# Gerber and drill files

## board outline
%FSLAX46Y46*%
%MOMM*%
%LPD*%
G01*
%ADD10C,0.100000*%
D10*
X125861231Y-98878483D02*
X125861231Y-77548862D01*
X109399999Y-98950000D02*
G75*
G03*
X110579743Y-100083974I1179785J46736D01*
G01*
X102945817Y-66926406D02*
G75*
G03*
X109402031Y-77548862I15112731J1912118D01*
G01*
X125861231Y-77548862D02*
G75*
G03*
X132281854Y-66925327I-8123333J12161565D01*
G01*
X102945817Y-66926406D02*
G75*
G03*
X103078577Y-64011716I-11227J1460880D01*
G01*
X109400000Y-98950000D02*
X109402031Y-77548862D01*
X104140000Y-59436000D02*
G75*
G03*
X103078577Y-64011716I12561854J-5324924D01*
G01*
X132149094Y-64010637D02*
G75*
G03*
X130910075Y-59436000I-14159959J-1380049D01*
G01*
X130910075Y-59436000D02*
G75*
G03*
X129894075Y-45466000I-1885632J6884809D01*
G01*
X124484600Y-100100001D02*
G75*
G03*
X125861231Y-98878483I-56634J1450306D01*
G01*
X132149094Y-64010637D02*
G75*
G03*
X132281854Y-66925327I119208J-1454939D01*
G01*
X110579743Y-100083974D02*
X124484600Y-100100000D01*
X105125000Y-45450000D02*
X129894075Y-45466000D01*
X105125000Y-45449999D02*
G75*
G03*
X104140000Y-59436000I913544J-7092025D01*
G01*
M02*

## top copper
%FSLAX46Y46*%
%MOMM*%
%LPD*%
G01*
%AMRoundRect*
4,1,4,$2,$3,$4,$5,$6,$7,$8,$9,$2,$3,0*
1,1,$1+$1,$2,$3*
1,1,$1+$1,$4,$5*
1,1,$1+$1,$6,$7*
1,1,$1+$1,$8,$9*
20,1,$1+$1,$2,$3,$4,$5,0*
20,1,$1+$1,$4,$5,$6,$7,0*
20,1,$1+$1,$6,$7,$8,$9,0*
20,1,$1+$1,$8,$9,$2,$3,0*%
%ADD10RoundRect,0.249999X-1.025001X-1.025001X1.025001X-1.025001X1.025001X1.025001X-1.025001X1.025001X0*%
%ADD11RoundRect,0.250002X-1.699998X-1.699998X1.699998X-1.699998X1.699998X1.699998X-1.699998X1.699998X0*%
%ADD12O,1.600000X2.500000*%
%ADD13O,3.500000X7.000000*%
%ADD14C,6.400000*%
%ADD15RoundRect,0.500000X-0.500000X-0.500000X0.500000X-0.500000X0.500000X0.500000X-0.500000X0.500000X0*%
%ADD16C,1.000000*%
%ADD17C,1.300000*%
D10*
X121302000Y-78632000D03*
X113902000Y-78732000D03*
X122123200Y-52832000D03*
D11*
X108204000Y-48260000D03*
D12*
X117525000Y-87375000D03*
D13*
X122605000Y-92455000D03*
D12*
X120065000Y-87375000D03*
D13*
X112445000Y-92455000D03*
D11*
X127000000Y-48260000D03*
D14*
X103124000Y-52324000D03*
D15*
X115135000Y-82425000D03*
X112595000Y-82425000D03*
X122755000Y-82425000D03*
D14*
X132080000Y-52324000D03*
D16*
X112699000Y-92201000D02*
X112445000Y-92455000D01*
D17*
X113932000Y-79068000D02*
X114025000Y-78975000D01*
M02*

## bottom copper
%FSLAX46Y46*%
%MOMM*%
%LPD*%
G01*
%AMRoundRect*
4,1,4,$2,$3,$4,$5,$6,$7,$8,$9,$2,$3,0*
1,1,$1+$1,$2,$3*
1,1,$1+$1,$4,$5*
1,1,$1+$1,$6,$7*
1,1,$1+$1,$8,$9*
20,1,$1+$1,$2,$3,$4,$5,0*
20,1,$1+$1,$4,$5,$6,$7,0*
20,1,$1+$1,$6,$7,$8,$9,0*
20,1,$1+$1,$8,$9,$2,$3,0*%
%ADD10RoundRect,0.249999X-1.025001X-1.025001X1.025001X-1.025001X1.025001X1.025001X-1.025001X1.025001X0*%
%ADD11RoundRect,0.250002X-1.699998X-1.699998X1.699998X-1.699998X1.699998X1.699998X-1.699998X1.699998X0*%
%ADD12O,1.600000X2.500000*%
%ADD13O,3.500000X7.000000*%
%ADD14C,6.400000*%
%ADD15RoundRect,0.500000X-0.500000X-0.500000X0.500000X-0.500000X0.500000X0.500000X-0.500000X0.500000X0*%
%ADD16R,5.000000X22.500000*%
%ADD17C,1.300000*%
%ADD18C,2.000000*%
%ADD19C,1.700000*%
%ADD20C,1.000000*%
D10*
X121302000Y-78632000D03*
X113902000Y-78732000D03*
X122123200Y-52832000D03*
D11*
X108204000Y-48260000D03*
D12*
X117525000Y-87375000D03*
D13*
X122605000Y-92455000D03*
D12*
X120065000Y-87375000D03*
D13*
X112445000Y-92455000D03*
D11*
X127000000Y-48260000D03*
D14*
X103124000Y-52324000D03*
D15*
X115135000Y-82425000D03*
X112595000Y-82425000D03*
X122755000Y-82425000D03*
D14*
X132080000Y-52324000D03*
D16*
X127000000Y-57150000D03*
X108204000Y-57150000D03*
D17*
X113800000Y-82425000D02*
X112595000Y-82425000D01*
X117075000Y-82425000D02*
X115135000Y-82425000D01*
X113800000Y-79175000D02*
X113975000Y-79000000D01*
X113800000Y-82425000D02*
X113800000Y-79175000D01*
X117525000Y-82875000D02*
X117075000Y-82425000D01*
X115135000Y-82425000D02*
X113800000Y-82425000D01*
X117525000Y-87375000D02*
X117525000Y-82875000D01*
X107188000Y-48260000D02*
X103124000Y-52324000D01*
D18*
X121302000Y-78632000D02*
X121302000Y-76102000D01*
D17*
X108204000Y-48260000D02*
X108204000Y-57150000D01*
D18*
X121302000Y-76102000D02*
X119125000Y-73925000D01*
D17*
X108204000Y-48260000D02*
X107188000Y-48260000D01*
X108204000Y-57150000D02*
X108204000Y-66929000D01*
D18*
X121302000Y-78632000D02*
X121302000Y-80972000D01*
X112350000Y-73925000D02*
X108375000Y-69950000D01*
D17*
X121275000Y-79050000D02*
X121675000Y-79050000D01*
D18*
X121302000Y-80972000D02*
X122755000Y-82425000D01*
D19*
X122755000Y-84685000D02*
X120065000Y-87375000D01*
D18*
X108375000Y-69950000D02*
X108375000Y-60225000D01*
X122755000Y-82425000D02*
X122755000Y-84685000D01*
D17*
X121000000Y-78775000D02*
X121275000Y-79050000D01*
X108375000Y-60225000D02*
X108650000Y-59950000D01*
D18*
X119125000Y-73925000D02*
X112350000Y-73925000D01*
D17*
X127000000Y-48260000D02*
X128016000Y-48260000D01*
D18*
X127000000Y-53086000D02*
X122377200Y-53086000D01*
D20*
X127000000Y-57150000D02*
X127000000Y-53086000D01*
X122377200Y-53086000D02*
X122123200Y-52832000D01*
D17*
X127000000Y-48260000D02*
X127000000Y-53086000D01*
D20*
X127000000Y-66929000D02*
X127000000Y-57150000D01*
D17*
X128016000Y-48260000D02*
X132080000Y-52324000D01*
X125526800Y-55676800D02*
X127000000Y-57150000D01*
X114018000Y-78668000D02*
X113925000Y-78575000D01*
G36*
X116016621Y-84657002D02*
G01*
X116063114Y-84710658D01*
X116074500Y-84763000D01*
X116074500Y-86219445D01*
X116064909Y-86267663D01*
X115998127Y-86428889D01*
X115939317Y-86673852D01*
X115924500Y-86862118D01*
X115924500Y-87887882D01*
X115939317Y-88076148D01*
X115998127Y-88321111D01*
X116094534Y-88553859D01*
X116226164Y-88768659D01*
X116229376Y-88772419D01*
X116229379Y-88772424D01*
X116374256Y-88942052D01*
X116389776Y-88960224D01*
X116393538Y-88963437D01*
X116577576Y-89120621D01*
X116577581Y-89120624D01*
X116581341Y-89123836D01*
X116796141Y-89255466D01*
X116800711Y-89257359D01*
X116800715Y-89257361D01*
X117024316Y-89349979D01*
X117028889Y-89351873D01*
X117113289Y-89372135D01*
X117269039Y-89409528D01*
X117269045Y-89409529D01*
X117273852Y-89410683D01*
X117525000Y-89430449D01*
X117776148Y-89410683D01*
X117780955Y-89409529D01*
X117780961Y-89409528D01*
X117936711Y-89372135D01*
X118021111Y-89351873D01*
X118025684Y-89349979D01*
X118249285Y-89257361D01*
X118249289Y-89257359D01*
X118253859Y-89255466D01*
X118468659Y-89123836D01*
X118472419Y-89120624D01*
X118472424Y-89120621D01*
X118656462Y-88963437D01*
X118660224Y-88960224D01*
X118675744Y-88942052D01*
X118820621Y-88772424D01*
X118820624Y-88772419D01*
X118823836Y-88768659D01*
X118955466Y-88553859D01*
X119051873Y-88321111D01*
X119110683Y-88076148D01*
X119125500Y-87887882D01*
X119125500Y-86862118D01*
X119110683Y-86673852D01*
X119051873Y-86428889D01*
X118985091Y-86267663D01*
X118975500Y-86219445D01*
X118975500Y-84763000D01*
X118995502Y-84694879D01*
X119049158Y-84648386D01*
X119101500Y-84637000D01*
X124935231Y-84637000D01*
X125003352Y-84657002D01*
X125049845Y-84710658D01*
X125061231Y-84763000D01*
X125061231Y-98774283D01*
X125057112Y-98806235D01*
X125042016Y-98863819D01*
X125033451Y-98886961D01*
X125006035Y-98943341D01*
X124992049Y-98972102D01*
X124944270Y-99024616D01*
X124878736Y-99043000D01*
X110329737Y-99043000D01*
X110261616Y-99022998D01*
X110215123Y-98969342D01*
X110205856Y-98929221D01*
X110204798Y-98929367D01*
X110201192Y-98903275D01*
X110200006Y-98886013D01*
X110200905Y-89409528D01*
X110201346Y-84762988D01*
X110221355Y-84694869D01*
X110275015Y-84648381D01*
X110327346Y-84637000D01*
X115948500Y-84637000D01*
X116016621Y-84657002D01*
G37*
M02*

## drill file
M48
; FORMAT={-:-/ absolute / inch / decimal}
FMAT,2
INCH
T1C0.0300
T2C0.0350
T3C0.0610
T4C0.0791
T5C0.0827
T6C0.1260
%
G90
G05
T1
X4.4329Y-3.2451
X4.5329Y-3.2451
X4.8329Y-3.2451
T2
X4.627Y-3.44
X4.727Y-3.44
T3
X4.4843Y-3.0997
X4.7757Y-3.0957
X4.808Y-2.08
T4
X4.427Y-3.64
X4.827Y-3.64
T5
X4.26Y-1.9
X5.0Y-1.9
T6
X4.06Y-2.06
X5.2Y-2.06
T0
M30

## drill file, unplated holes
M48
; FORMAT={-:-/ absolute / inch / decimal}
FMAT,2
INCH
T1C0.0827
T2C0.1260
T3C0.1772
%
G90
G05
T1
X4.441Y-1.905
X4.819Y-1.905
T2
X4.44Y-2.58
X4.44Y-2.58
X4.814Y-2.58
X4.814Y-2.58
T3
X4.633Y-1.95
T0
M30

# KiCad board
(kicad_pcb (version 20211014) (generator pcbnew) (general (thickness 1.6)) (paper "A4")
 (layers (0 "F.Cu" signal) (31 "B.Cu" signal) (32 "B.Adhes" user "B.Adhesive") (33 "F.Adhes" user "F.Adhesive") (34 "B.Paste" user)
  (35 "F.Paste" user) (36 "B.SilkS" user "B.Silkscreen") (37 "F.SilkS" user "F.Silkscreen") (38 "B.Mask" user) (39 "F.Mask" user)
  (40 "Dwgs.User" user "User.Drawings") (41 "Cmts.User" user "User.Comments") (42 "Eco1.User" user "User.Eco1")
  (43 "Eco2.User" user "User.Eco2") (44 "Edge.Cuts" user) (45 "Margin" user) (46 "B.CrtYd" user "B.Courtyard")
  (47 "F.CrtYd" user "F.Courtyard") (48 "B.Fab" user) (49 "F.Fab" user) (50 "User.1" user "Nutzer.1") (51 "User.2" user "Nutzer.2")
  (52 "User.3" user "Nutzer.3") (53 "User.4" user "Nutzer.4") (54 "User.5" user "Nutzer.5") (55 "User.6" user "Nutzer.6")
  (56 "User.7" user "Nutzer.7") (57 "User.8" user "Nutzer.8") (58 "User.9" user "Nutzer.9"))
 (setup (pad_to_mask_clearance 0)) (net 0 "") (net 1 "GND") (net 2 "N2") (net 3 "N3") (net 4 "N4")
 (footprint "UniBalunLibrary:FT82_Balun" (layer "F.Cu") (at 117.602 65.532)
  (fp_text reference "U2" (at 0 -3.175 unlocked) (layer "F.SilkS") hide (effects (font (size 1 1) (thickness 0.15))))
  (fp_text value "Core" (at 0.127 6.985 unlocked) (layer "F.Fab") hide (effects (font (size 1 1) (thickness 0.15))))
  (pad "" np_thru_hole circle (at 4.6736 0) (size 3.2 3.2) (drill 3.2) (layers *.Cu *.Mask))
  (pad "" np_thru_hole circle (at -4.826 0) (size 3.2 3.2) (drill 3.2) (layers *.Cu *.Mask))
  (pad "" np_thru_hole circle (at -4.826 0) (size 3.2 3.2) (drill 3.2) (layers *.Cu *.Mask))
  (pad "" np_thru_hole circle (at 4.6736 0) (size 3.2 3.2) (drill 3.2) (layers *.Cu *.Mask))
  (pad "1" thru_hole roundrect (at 3.7 13.1) (size 2.55 2.55) (drill 1.55) (layers *.Cu *.Mask) (roundrect_rratio 0.09803882353)
   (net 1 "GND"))
  (pad "4" thru_hole roundrect (at -3.7 13.2) (size 2.55 2.55) (drill 1.55) (layers *.Cu *.Mask) (roundrect_rratio 0.09803882353)
   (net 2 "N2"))
  (pad "5" thru_hole roundrect (at 4.5212 -12.7) (size 2.55 2.55) (drill 1.55) (layers *.Cu *.Mask) (roundrect_rratio 0.09803882353)
   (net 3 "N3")))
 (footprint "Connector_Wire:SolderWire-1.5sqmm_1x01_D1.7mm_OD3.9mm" (layer "F.Cu") (at 108.204 48.26)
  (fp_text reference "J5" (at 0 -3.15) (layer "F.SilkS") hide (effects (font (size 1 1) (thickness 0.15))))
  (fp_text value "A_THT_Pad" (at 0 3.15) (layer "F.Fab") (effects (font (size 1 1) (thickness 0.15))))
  (pad "1" thru_hole roundrect (at 0 0) (size 3.9 3.9) (drill 2.1) (layers *.Cu *.Mask) (roundrect_rratio 0.06410307692) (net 1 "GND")))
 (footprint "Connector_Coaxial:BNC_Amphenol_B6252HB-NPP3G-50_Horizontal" (layer "F.Cu") (at 117.525 87.375 180)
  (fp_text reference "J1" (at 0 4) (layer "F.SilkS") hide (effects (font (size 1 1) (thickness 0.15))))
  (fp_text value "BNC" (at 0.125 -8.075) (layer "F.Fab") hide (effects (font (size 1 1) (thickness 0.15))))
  (pad "1" thru_hole oval (at 0 0 180) (size 1.6 2.5) (drill 0.89) (layers *.Cu *.Mask) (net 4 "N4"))
  (pad "2" thru_hole oval (at -5.08 -5.08 180) (size 3.5 7) (drill 2.01) (layers *.Cu *.Mask) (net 1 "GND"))
  (pad "2" thru_hole oval (at -2.54 0 180) (size 1.6 2.5) (drill 0.89) (layers *.Cu *.Mask) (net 1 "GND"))
  (pad "2" thru_hole oval (at 5.08 -5.08 180) (size 3.5 7) (drill 2.01) (layers *.Cu *.Mask) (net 1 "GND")))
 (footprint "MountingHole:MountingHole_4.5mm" (layer "F.Cu") (at 117.6782 49.53)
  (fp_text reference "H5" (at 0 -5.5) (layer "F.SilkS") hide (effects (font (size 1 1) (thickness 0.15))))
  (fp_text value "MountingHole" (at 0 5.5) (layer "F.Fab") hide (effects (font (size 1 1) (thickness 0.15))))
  (pad "" np_thru_hole circle (at 0 0) (size 4.5 4.5) (drill 4.5) (layers *.Cu *.Mask)))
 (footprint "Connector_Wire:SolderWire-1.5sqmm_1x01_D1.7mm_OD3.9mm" (layer "F.Cu") (at 127 48.26)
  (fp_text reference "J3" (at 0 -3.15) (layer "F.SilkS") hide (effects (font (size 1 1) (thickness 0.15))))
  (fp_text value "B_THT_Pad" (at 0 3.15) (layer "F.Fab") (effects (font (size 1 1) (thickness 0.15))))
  (pad "1" thru_hole roundrect (at 0 0) (size 3.9 3.9) (drill 2.1) (layers *.Cu *.Mask) (roundrect_rratio 0.06410307692) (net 3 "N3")))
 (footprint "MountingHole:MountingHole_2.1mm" (layer "F.Cu") (at 112.8014 48.387)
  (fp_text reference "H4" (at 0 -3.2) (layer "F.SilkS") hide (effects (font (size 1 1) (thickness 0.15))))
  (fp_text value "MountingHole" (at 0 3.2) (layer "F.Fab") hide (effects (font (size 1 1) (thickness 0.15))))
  (pad "" np_thru_hole circle (at 0 0) (size 2.1 2.1) (drill 2.1) (layers *.Cu *.Mask)))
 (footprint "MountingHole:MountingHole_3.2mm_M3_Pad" (layer "F.Cu") (at 103.124 52.324)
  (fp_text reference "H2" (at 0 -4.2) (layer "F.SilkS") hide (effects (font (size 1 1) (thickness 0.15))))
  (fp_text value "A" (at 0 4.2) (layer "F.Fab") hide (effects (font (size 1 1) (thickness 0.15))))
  (pad "1" thru_hole circle (at 0 0) (size 6.4 6.4) (drill 3.2) (layers *.Cu *.Mask) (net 1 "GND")))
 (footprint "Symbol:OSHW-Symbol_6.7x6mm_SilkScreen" (layer "F.Cu") (at 117.4 68.7)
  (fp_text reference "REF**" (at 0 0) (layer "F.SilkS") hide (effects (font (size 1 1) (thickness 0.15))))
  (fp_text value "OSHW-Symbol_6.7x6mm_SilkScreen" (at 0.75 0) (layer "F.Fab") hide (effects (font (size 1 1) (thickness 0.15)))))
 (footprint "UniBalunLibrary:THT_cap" (layer "F.Cu") (at 117.675 82.425)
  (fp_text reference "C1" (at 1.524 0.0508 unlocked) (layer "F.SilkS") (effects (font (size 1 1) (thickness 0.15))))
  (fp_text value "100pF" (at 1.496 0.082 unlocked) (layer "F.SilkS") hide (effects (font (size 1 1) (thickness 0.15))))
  (pad "1" thru_hole roundrect (at -2.54 0) (size 2 2) (drill 0.762) (layers *.Cu *.Mask) (roundrect_rratio 0.25) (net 4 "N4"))
  (pad "1" thru_hole roundrect (at -5.08 0) (size 2 2) (drill 0.762) (layers *.Cu *.Mask) (roundrect_rratio 0.25) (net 4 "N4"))
  (pad "2" thru_hole roundrect (at 5.08 0) (size 2 2) (drill 0.762) (layers *.Cu *.Mask) (roundrect_rratio 0.25) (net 1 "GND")))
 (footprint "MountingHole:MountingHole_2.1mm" (layer "F.Cu") (at 122.4026 48.387)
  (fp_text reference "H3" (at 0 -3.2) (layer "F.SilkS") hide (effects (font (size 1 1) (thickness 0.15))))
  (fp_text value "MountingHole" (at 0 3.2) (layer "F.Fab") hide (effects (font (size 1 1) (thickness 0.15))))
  (pad "" np_thru_hole circle (at 0 0) (size 2.1 2.1) (drill 2.1) (layers *.Cu *.Mask)))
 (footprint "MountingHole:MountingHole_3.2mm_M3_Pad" (layer "F.Cu") (at 132.08 52.324)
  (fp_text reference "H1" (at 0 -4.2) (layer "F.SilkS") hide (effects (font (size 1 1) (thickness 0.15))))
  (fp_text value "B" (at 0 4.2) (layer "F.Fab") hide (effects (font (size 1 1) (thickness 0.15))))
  (pad "1" thru_hole circle (at 0 0) (size 6.4 6.4) (drill 3.2) (layers *.Cu *.Mask) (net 3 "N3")))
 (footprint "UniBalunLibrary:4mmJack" (layer "B.Cu") (at 127.254 56.896 90)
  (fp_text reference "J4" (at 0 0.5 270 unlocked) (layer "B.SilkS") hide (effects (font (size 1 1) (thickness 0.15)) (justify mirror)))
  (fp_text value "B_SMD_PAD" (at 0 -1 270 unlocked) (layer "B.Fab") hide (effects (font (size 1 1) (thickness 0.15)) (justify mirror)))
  (pad "1" smd rect (at -0.254 -0.254 90) (size 22.5 5) (layers "B.Cu" "B.Mask") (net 3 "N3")))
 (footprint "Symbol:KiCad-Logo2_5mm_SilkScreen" (layer "B.Cu") (at 117.729 58.547 180)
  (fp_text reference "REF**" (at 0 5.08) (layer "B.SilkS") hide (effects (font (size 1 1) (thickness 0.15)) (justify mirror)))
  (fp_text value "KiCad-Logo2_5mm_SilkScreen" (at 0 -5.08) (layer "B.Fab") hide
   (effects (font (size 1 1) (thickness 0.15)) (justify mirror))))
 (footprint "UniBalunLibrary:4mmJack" (layer "B.Cu") (at 108.458 56.896 90)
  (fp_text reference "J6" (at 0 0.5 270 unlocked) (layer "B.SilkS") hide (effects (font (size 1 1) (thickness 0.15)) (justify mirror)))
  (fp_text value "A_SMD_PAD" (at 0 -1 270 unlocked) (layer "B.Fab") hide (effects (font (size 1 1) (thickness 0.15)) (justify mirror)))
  (pad "1" smd rect (at -0.254 -0.254 90) (size 22.5 5) (layers "B.Cu" "B.Mask") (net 1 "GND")))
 (gr_line (start 125.861231 98.878483) (end 125.861231 77.548862) (layer "Edge.Cuts") (width 0.1))
 (gr_arc (start 110.579743 100.083974) (mid 109.761572 99.754501) (end 109.4 98.95) (layer "Edge.Cuts") (width 0.1))
 (gr_arc (start 109.402031 77.548862) (mid 105.04112 72.92614) (end 102.945817 66.926406) (layer "Edge.Cuts") (width 0.1))
 (gr_arc (start 132.281854 66.925327) (mid 130.254542 72.952072) (end 125.861231 77.548862) (layer "Edge.Cuts") (width 0.1))
 (gr_arc (start 103.078577 64.011716) (mid 104.394 65.532) (end 102.945817 66.926406) (layer "Edge.Cuts") (width 0.1))
 (gr_line (start 109.4 98.95) (end 109.402031 77.548862) (layer "Edge.Cuts") (width 0.1))
 (gr_arc (start 103.078577 64.011716) (mid 103.410896 61.677837) (end 104.14 59.436) (layer "Edge.Cuts") (width 0.1))
 (gr_arc (start 130.910075 59.436) (mid 131.721418 61.671361) (end 132.149094 64.010637) (layer "Edge.Cuts") (width 0.1))
 (gr_arc (start 129.894075 45.466) (mid 136.144 52.033405) (end 130.910075 59.436) (layer "Edge.Cuts") (width 0.1))
 (gr_arc (start 125.861231 98.878483) (mid 125.391281 99.735336) (end 124.4846 100.1) (layer "Edge.Cuts") (width 0.1))
 (gr_arc (start 132.281854 66.925327) (mid 130.81 65.532) (end 132.149094 64.010637) (layer "Edge.Cuts") (width 0.1))
 (gr_line (start 110.579743 100.083974) (end 124.4846 100.1) (layer "Edge.Cuts") (width 0.1))
 (gr_line (start 105.125 45.45) (end 129.894075 45.466) (layer "Edge.Cuts") (width 0.1))
 (gr_arc (start 104.14 59.436) (mid 98.905591 52.039668) (end 105.125 45.45) (layer "Edge.Cuts") (width 0.1))
 (segment (start 113.8 82.425) (end 112.595 82.425) (width 1.3) (layer "B.Cu") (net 4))
 (segment (start 117.075 82.425) (end 115.135 82.425) (width 1.3) (layer "B.Cu") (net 4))
 (segment (start 113.8 79.175) (end 113.975 79) (width 1.3) (layer "B.Cu") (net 4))
 (segment (start 113.8 82.425) (end 113.8 79.175) (width 1.3) (layer "B.Cu") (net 4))
 (segment (start 117.525 82.875) (end 117.075 82.425) (width 1.3) (layer "B.Cu") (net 4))
 (segment (start 115.135 82.425) (end 113.8 82.425) (width 1.3) (layer "B.Cu") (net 4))
 (segment (start 117.525 87.375) (end 117.525 82.875) (width 1.3) (layer "B.Cu") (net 4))
 (segment (start 112.699 92.201) (end 112.445 92.455) (width 1) (layer "F.Cu") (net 1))
 (segment (start 107.188 48.26) (end 103.124 52.324) (width 1.3) (layer "B.Cu") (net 1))
 (segment (start 121.302 78.632) (end 121.302 76.102) (width 2) (layer "B.Cu") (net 1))
 (segment (start 108.204 48.26) (end 108.204 57.15) (width 1.3) (layer "B.Cu") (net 1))
 (segment (start 121.302 76.102) (end 119.125 73.925) (width 2) (layer "B.Cu") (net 1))
 (segment (start 108.204 48.26) (end 107.188 48.26) (width 1.3) (layer "B.Cu") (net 1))
 (segment (start 108.204 57.15) (end 108.204 66.929) (width 1.3) (layer "B.Cu") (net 1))
 (segment (start 121.302 78.632) (end 121.302 80.972) (width 2) (layer "B.Cu") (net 1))
 (segment (start 112.35 73.925) (end 108.375 69.95) (width 2) (layer "B.Cu") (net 1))
 (segment (start 121.275 79.05) (end 121.675 79.05) (width 1.3) (layer "B.Cu") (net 1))
 (segment (start 121.302 80.972) (end 122.755 82.425) (width 2) (layer "B.Cu") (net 1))
 (segment (start 122.755 84.685) (end 120.065 87.375) (width 1.7) (layer "B.Cu") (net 1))
 (segment (start 108.375 69.95) (end 108.375 60.225) (width 2) (layer "B.Cu") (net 1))
 (segment (start 122.755 82.425) (end 122.755 84.685) (width 2) (layer "B.Cu") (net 1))
 (segment (start 121 78.775) (end 121.275 79.05) (width 1.3) (layer "B.Cu") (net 1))
 (segment (start 108.375 60.225) (end 108.65 59.95) (width 1.3) (layer "B.Cu") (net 1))
 (segment (start 119.125 73.925) (end 112.35 73.925) (width 2) (layer "B.Cu") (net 1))
 (segment (start 127 48.26) (end 128.016 48.26) (width 1.3) (layer "B.Cu") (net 3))
 (segment (start 127 53.086) (end 122.3772 53.086) (width 2) (layer "B.Cu") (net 3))
 (segment (start 127 57.15) (end 127 53.086) (width 1) (layer "B.Cu") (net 3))
 (segment (start 122.3772 53.086) (end 122.1232 52.832) (width 1) (layer "B.Cu") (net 3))
 (segment (start 127 48.26) (end 127 53.086) (width 1.3) (layer "B.Cu") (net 3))
 (segment (start 127 66.929) (end 127 57.15) (width 1) (layer "B.Cu") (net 3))
 (segment (start 128.016 48.26) (end 132.08 52.324) (width 1.3) (layer "B.Cu") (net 3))
 (segment (start 125.5268 55.6768) (end 127 57.15) (width 1.3) (layer "B.Cu") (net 3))
 (segment (start 113.932 79.068) (end 114.025 78.975) (width 1.3) (layer "F.Cu") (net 2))
 (segment (start 114.018 78.668) (end 113.925 78.575) (width 1.3) (layer "B.Cu") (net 2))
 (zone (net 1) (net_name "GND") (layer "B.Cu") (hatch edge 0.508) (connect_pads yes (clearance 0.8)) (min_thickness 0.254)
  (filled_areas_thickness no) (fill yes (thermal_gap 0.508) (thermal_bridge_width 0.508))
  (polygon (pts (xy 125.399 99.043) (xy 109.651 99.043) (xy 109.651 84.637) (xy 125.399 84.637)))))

